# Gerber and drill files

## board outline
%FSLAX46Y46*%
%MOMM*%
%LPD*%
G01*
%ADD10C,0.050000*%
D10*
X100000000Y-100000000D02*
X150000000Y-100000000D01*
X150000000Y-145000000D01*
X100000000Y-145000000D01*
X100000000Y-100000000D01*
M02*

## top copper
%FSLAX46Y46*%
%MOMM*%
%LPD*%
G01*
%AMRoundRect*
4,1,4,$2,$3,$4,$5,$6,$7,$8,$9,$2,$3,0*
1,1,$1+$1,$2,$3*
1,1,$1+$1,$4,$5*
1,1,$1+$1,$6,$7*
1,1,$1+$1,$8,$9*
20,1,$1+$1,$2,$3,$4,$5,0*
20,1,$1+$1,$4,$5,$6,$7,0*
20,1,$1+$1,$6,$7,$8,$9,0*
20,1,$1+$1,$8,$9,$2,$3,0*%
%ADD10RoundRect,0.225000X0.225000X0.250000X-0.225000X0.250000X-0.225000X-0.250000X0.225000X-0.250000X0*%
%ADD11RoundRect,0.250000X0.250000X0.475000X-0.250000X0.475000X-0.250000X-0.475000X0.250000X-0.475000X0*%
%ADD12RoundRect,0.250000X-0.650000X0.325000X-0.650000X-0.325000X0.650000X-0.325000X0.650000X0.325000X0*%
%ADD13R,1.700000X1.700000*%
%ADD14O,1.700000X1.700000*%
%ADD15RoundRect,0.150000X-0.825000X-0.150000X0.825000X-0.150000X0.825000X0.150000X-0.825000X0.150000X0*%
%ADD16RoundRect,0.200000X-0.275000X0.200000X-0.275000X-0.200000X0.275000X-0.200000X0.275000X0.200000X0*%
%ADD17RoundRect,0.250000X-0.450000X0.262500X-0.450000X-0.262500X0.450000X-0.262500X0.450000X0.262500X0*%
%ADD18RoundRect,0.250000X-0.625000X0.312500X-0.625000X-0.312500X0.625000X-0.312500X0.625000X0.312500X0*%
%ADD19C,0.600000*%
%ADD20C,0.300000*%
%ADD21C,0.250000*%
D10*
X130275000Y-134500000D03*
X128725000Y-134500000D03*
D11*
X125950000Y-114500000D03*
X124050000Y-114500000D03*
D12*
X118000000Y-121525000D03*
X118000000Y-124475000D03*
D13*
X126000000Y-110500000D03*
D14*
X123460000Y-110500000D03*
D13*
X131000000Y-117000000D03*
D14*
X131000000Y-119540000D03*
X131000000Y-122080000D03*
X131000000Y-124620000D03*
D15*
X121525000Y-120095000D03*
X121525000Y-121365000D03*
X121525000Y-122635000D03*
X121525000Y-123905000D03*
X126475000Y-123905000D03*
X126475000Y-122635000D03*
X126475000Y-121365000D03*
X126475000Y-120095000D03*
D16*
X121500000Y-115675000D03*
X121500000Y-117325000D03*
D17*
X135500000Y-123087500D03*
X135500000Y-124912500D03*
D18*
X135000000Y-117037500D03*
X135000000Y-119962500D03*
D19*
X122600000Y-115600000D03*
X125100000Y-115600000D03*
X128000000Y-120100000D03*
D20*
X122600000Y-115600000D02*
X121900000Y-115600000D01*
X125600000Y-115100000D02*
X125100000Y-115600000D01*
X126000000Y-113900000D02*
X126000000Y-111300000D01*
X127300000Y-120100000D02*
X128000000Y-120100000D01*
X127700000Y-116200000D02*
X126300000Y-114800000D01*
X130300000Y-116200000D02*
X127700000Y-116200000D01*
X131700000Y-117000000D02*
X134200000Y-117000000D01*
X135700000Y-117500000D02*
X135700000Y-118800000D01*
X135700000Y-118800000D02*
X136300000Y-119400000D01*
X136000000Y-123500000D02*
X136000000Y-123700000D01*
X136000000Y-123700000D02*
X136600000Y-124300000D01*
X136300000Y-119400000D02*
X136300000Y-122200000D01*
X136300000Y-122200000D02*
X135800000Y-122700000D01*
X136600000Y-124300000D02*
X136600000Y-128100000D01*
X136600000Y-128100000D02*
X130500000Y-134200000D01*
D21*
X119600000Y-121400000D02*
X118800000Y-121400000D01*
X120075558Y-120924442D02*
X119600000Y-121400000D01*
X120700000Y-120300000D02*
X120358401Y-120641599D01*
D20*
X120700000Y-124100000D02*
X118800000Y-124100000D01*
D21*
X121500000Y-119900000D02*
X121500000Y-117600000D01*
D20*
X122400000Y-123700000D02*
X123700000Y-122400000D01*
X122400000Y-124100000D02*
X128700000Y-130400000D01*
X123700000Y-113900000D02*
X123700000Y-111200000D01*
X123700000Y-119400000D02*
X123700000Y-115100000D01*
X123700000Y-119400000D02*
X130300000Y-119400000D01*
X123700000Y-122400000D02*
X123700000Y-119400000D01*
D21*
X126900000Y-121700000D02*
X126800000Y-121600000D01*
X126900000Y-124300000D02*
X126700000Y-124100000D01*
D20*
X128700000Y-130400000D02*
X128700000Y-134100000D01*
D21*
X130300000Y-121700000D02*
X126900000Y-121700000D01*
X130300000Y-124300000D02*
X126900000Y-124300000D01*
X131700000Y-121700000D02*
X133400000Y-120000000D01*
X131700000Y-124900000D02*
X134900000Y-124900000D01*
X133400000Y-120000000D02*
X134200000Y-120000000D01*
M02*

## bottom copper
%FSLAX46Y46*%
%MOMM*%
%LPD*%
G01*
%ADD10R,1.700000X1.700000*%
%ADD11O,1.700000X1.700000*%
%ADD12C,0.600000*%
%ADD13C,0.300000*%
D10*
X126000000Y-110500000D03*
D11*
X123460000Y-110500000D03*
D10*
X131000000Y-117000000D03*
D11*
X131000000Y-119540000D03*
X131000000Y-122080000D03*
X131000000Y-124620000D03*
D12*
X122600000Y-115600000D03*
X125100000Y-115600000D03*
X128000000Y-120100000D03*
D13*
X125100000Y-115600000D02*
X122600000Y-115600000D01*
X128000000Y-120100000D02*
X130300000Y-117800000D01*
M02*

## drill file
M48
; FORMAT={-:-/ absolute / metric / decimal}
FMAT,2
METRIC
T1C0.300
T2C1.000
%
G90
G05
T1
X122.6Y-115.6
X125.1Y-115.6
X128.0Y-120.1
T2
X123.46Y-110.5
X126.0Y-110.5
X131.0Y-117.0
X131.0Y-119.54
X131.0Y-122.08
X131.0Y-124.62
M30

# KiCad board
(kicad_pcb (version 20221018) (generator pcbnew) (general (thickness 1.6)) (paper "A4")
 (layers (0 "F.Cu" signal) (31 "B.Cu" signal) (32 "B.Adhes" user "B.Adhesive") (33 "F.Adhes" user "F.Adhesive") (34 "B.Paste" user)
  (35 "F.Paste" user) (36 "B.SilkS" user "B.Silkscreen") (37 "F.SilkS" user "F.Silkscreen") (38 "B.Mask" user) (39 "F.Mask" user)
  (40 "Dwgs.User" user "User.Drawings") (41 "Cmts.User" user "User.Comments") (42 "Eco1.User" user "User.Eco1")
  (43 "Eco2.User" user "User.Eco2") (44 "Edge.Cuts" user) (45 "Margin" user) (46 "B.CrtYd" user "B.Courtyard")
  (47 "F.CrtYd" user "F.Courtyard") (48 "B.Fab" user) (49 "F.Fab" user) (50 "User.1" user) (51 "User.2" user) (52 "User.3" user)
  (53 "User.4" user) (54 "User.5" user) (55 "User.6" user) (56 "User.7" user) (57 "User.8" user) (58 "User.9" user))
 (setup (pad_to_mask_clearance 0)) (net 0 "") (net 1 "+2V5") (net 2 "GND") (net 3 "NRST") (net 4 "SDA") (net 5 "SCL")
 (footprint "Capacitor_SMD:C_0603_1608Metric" (layer "F.Cu") (at 129.5 134.5 180)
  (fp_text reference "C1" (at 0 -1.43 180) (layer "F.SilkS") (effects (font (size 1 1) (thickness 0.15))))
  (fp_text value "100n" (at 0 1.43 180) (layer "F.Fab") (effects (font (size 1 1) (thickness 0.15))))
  (pad "1" smd roundrect (at -0.775 0 180) (size 0.9 0.95) (layers "F.Cu" "F.Paste" "F.Mask") (roundrect_rratio 0.25) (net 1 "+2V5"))
  (pad "2" smd roundrect (at 0.775 0 180) (size 0.9 0.95) (layers "F.Cu" "F.Paste" "F.Mask") (roundrect_rratio 0.25) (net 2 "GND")))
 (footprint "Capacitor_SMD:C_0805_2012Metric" (layer "F.Cu") (at 125 114.5 180)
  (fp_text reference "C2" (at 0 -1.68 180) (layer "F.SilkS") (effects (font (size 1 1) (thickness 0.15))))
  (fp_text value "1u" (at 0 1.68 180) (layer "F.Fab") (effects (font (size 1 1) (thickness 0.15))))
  (pad "1" smd roundrect (at -0.95 0 180) (size 1 1.45) (layers "F.Cu" "F.Paste" "F.Mask") (roundrect_rratio 0.25) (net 1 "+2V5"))
  (pad "2" smd roundrect (at 0.95 0 180) (size 1 1.45) (layers "F.Cu" "F.Paste" "F.Mask") (roundrect_rratio 0.25) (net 2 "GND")))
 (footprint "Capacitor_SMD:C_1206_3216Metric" (layer "F.Cu") (at 118 123 -90)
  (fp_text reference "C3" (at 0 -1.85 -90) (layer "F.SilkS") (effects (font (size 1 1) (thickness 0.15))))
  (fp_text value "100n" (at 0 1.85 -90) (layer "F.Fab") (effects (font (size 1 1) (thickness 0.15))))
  (pad "1" smd roundrect (at -1.475 0 270) (size 1.15 1.8) (layers "F.Cu" "F.Paste" "F.Mask") (roundrect_rratio 0.217391) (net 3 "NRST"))
  (pad "2" smd roundrect (at 1.475 0 270) (size 1.15 1.8) (layers "F.Cu" "F.Paste" "F.Mask") (roundrect_rratio 0.217391) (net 2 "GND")))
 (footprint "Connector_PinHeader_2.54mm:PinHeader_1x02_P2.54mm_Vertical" (layer "F.Cu") (at 126 110.5 -90)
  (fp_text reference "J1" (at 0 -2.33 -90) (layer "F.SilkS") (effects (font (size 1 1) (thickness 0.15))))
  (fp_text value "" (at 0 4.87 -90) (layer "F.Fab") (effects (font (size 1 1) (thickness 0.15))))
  (pad "1" thru_hole rect (at 0 0 270) (size 1.7 1.7) (drill 1) (layers "*.Cu" "*.Mask") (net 1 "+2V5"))
  (pad "2" thru_hole oval (at 0 2.54 270) (size 1.7 1.7) (drill 1) (layers "*.Cu" "*.Mask") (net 2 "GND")))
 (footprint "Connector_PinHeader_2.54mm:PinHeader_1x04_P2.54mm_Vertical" (layer "F.Cu") (at 131 117)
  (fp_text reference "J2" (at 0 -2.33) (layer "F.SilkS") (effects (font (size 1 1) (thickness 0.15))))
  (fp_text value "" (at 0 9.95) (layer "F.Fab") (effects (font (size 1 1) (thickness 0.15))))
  (pad "1" thru_hole rect (at 0 0) (size 1.7 1.7) (drill 1) (layers "*.Cu" "*.Mask") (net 1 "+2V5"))
  (pad "2" thru_hole oval (at 0 2.54) (size 1.7 1.7) (drill 1) (layers "*.Cu" "*.Mask") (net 2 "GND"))
  (pad "3" thru_hole oval (at 0 5.08) (size 1.7 1.7) (drill 1) (layers "*.Cu" "*.Mask") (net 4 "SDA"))
  (pad "4" thru_hole oval (at 0 7.62) (size 1.7 1.7) (drill 1) (layers "*.Cu" "*.Mask") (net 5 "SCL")))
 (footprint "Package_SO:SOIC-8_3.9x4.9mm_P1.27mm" (layer "F.Cu") (at 124 122)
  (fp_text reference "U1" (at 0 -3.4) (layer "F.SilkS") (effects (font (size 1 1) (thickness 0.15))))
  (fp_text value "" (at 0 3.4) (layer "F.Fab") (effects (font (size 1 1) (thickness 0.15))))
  (pad "1" smd roundrect (at -2.475 -1.905) (size 1.95 0.6) (layers "F.Cu" "F.Paste" "F.Mask") (roundrect_rratio 0.25) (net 3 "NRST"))
  (pad "2" smd roundrect (at -2.475 -0.635) (size 1.95 0.6) (layers "F.Cu" "F.Paste" "F.Mask") (roundrect_rratio 0.25))
  (pad "3" smd roundrect (at -2.475 0.635) (size 1.95 0.6) (layers "F.Cu" "F.Paste" "F.Mask") (roundrect_rratio 0.25))
  (pad "4" smd roundrect (at -2.475 1.905) (size 1.95 0.6) (layers "F.Cu" "F.Paste" "F.Mask") (roundrect_rratio 0.25) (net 2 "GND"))
  (pad "5" smd roundrect (at 2.475 1.905) (size 1.95 0.6) (layers "F.Cu" "F.Paste" "F.Mask") (roundrect_rratio 0.25) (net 5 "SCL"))
  (pad "6" smd roundrect (at 2.475 0.635) (size 1.95 0.6) (layers "F.Cu" "F.Paste" "F.Mask") (roundrect_rratio 0.25))
  (pad "7" smd roundrect (at 2.475 -0.635) (size 1.95 0.6) (layers "F.Cu" "F.Paste" "F.Mask") (roundrect_rratio 0.25) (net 4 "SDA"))
  (pad "8" smd roundrect (at 2.475 -1.905) (size 1.95 0.6) (layers "F.Cu" "F.Paste" "F.Mask") (roundrect_rratio 0.25) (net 1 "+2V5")))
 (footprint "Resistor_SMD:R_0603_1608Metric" (layer "F.Cu") (at 121.5 116.5 -90)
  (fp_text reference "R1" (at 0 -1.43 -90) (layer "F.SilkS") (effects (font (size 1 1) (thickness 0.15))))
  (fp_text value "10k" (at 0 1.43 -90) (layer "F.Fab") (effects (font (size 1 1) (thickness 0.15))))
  (pad "1" smd roundrect (at -0.825 0 270) (size 0.8 0.95) (layers "F.Cu" "F.Paste" "F.Mask") (roundrect_rratio 0.25) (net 1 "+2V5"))
  (pad "2" smd roundrect (at 0.825 0 270) (size 0.8 0.95) (layers "F.Cu" "F.Paste" "F.Mask") (roundrect_rratio 0.25) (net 3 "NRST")))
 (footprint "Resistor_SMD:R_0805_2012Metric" (layer "F.Cu") (at 135.5 124 -90)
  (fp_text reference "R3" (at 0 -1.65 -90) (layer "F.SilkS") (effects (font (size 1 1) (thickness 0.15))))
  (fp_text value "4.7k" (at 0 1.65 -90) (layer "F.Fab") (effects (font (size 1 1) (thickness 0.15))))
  (pad "1" smd roundrect (at -0.9125 0 270) (size 1.025 1.4) (layers "F.Cu" "F.Paste" "F.Mask") (roundrect_rratio 0.243902) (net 1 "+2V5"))
  (pad "2" smd roundrect (at 0.9125 0 270) (size 1.025 1.4) (layers "F.Cu" "F.Paste" "F.Mask") (roundrect_rratio 0.243902) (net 5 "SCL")))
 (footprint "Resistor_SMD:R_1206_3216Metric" (layer "F.Cu") (at 135 118.5 -90)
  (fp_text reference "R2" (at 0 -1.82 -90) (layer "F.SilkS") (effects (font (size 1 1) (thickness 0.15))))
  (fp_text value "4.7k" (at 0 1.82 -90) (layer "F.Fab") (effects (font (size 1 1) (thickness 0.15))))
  (pad "1" smd roundrect (at -1.4625 0 270) (size 1.125 1.75) (layers "F.Cu" "F.Paste" "F.Mask") (roundrect_rratio 0.222222) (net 1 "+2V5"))
  (pad "2" smd roundrect (at 1.4625 0 270) (size 1.125 1.75) (layers "F.Cu" "F.Paste" "F.Mask") (roundrect_rratio 0.222222) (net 4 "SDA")))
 (gr_rect (start 100 100) (end 150 145) (stroke (width 0.05) (type default)) (fill none) (layer "Edge.Cuts"))
 (segment (start 122.6 115.6) (end 121.9 115.6) (width 0.3) (layer "F.Cu") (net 1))
 (segment (start 125.6 115.1) (end 125.1 115.6) (width 0.3) (layer "F.Cu") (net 1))
 (segment (start 126 113.9) (end 126 111.3) (width 0.3) (layer "F.Cu") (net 1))
 (segment (start 127.3 120.1) (end 128 120.1) (width 0.3) (layer "F.Cu") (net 1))
 (segment (start 127.7 116.2) (end 126.3 114.8) (width 0.3) (layer "F.Cu") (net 1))
 (segment (start 130.3 116.2) (end 127.7 116.2) (width 0.3) (layer "F.Cu") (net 1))
 (segment (start 131.7 117) (end 134.2 117) (width 0.3) (layer "F.Cu") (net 1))
 (segment (start 135.7 117.5) (end 135.7 118.8) (width 0.3) (layer "F.Cu") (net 1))
 (segment (start 135.7 118.8) (end 136.3 119.4) (width 0.3) (layer "F.Cu") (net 1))
 (segment (start 136 123.5) (end 136 123.7) (width 0.3) (layer "F.Cu") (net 1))
 (segment (start 136 123.7) (end 136.6 124.3) (width 0.3) (layer "F.Cu") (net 1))
 (segment (start 136.3 119.4) (end 136.3 122.2) (width 0.3) (layer "F.Cu") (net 1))
 (segment (start 136.3 122.2) (end 135.8 122.7) (width 0.3) (layer "F.Cu") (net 1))
 (segment (start 136.6 124.3) (end 136.6 128.1) (width 0.3) (layer "F.Cu") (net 1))
 (segment (start 136.6 128.1) (end 130.5 134.2) (width 0.3) (layer "F.Cu") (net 1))
 (via (at 122.6 115.6) (size 0.6) (drill 0.3) (layers "F.Cu" "B.Cu") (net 1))
 (via (at 125.1 115.6) (size 0.6) (drill 0.3) (layers "F.Cu" "B.Cu") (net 1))
 (via (at 128 120.1) (size 0.6) (drill 0.3) (layers "F.Cu" "B.Cu") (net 1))
 (segment (start 119.6 121.4) (end 118.8 121.4) (width 0.25) (layer "F.Cu") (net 3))
 (segment (start 120.075558 120.924442) (end 119.6 121.4) (width 0.25) (layer "F.Cu") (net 3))
 (segment (start 120.7 120.3) (end 120.358401 120.641599) (width 0.25) (layer "F.Cu") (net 3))
 (segment (start 120.7 124.1) (end 118.8 124.1) (width 0.3) (layer "F.Cu") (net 2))
 (segment (start 121.5 119.9) (end 121.5 117.6) (width 0.25) (layer "F.Cu") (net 3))
 (segment (start 122.4 123.7) (end 123.7 122.4) (width 0.3) (layer "F.Cu") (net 2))
 (segment (start 122.4 124.1) (end 128.7 130.4) (width 0.3) (layer "F.Cu") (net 2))
 (segment (start 123.7 113.9) (end 123.7 111.2) (width 0.3) (layer "F.Cu") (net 2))
 (segment (start 123.7 119.4) (end 123.7 115.1) (width 0.3) (layer "F.Cu") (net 2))
 (segment (start 123.7 119.4) (end 130.3 119.4) (width 0.3) (layer "F.Cu") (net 2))
 (segment (start 123.7 122.4) (end 123.7 119.4) (width 0.3) (layer "F.Cu") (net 2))
 (segment (start 125.1 115.6) (end 122.6 115.6) (width 0.3) (layer "B.Cu") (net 1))
 (segment (start 126.9 121.7) (end 126.8 121.6) (width 0.25) (layer "F.Cu") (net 4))
 (segment (start 126.9 124.3) (end 126.7 124.1) (width 0.25) (layer "F.Cu") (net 5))
 (segment (start 128 120.1) (end 130.3 117.8) (width 0.3) (layer "B.Cu") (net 1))
 (segment (start 128.7 130.4) (end 128.7 134.1) (width 0.3) (layer "F.Cu") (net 2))
 (segment (start 130.3 121.7) (end 126.9 121.7) (width 0.25) (layer "F.Cu") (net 4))
 (segment (start 130.3 124.3) (end 126.9 124.3) (width 0.25) (layer "F.Cu") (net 5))
 (segment (start 131.7 121.7) (end 133.4 120) (width 0.25) (layer "F.Cu") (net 4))
 (segment (start 131.7 124.9) (end 134.9 124.9) (width 0.25) (layer "F.Cu") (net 5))
 (segment (start 133.4 120) (end 134.2 120) (width 0.25) (layer "F.Cu") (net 4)))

